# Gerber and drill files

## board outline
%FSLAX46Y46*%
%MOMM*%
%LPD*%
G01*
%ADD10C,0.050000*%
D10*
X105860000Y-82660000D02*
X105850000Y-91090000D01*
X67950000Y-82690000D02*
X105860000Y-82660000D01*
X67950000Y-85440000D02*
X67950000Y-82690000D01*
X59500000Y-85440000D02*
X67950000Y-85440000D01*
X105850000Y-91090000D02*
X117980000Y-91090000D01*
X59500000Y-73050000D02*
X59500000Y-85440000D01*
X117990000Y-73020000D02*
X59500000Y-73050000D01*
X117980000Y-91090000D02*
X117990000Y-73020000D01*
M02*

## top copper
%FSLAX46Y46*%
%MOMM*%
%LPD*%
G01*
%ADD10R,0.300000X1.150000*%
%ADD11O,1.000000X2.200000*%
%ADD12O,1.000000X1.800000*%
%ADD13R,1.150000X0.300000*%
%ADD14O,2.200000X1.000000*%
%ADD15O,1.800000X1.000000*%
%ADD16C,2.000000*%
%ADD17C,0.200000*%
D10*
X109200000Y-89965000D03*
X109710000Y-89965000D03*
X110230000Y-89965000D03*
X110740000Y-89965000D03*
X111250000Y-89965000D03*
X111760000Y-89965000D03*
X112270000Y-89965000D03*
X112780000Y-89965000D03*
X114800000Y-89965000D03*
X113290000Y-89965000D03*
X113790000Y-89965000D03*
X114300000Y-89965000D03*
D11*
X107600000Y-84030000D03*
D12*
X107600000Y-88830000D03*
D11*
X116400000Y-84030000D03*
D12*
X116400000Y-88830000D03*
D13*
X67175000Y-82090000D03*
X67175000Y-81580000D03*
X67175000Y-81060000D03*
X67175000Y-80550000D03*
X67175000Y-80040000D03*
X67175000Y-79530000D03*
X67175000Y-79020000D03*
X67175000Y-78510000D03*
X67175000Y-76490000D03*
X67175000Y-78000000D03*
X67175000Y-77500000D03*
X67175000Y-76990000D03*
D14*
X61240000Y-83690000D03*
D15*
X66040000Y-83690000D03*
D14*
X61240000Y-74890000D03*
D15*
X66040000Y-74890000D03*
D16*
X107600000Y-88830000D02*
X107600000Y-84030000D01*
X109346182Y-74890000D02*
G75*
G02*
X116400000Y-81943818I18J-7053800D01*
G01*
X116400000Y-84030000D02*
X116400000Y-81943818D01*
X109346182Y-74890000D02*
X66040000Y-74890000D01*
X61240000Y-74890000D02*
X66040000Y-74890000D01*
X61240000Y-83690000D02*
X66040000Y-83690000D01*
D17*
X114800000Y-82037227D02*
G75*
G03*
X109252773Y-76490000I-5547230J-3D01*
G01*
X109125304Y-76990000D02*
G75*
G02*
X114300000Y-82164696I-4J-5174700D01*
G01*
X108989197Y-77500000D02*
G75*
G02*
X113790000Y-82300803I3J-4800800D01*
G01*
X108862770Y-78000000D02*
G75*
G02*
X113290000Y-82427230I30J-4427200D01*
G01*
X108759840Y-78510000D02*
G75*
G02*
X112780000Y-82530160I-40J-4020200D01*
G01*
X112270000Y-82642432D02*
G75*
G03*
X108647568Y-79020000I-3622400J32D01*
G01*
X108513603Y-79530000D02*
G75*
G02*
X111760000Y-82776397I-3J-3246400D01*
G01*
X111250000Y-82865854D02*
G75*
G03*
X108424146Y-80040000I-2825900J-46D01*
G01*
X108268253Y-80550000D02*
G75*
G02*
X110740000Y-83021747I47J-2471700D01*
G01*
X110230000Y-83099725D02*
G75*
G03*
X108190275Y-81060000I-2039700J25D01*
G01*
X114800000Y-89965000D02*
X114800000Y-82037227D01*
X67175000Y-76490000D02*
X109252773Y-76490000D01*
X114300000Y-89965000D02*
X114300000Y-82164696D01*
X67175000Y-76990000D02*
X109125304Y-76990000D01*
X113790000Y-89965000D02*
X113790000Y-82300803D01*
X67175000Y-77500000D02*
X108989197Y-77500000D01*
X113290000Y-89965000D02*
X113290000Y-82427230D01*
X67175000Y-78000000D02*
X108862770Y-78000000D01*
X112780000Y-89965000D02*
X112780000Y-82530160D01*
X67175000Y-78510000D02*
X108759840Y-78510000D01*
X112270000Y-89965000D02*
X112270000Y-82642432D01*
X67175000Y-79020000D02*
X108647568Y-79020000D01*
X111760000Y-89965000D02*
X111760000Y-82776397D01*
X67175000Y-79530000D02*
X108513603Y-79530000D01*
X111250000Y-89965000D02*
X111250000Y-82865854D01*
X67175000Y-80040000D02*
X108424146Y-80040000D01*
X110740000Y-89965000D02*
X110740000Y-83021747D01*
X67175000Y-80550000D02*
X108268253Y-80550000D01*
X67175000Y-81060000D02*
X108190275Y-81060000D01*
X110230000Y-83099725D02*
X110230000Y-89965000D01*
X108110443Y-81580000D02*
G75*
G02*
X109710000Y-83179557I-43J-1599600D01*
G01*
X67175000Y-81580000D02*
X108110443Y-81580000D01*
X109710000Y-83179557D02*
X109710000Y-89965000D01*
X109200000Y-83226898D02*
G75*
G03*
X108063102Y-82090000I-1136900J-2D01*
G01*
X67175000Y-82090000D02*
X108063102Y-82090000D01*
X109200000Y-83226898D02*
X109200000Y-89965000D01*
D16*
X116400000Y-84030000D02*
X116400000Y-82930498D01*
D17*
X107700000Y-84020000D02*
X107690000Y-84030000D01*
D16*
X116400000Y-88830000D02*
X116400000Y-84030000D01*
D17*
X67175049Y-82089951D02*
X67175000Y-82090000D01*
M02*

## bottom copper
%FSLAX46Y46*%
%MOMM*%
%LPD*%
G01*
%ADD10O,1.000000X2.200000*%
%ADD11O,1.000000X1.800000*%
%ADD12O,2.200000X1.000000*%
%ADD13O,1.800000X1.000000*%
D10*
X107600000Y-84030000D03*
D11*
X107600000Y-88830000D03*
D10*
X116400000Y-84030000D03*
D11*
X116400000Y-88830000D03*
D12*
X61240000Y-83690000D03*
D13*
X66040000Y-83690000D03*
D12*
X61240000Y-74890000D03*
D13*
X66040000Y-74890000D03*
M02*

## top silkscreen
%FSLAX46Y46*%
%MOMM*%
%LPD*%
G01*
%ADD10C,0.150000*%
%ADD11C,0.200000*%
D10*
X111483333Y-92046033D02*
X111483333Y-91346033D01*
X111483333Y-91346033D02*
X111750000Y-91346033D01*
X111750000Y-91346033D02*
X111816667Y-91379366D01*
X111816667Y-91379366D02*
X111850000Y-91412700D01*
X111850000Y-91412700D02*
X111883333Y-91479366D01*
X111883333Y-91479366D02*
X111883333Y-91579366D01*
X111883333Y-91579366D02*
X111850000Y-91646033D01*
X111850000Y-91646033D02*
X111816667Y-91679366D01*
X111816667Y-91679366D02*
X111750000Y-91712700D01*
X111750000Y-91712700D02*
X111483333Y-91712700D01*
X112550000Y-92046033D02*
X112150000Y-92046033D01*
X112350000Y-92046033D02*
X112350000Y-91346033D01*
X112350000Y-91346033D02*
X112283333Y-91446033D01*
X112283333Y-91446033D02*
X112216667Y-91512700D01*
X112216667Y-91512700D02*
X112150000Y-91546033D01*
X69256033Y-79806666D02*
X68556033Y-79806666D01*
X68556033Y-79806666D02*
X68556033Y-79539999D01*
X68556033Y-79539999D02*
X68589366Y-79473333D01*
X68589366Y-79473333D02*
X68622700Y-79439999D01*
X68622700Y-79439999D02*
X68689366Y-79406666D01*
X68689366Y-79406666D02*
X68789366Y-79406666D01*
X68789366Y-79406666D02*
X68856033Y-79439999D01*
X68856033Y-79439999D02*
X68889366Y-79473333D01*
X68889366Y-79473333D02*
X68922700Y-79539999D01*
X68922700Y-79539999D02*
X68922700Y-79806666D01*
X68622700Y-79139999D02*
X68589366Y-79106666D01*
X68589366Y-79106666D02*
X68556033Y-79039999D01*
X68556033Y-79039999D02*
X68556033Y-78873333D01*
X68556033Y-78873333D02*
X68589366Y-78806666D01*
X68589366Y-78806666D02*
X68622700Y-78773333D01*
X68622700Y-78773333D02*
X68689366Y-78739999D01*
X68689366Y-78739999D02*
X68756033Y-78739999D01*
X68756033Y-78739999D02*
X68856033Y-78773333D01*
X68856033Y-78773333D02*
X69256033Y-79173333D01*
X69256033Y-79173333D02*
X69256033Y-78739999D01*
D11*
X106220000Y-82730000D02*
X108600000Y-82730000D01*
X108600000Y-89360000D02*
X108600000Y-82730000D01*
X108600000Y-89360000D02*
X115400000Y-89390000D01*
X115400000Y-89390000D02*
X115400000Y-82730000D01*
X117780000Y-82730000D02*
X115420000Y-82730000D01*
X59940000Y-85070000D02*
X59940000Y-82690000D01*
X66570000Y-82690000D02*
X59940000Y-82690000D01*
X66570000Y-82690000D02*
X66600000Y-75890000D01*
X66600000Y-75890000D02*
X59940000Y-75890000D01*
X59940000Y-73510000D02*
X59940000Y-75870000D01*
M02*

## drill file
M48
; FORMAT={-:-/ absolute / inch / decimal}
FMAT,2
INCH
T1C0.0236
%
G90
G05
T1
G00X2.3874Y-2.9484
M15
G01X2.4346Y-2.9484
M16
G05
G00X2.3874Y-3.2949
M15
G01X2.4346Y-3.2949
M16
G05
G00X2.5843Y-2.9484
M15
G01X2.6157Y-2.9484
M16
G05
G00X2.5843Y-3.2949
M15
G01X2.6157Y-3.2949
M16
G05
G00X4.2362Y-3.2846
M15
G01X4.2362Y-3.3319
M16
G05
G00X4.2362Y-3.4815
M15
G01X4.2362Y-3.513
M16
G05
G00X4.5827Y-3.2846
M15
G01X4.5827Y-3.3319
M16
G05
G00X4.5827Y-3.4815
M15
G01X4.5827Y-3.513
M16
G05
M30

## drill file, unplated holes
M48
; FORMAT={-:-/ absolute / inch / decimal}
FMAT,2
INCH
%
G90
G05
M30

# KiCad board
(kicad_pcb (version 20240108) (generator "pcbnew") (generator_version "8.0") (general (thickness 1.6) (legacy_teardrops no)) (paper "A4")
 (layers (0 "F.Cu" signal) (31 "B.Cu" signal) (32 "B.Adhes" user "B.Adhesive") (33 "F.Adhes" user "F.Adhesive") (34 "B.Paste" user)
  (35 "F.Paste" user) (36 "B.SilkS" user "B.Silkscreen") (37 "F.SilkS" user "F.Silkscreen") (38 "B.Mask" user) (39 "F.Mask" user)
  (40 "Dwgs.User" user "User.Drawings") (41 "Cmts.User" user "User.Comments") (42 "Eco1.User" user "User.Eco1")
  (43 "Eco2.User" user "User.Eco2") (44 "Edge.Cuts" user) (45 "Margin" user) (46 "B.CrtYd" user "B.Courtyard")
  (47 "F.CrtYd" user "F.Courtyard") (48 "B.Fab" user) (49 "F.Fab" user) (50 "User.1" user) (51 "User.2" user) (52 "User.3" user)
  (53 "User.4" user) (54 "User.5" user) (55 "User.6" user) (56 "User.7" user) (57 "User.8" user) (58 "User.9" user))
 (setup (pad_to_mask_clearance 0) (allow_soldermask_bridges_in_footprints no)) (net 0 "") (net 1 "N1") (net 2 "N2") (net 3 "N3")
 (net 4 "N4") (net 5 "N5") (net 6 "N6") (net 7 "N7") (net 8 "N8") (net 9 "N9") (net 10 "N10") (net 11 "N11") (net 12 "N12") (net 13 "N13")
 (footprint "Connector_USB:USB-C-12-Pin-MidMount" (layer "F.Cu") (at 112 82.73)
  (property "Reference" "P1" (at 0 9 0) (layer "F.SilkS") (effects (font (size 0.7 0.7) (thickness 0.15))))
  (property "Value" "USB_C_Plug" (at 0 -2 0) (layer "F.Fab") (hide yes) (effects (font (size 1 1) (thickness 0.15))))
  (fp_line (start -5.78 0) (end -3.4 0) (stroke (width 0.2) (type solid)) (layer "F.SilkS"))
  (fp_line (start -3.4 6.63) (end -3.4 0) (stroke (width 0.2) (type solid)) (layer "F.SilkS"))
  (fp_line (start -3.4 6.63) (end 3.4 6.66) (stroke (width 0.2) (type solid)) (layer "F.SilkS"))
  (fp_line (start 3.4 6.66) (end 3.4 0) (stroke (width 0.2) (type solid)) (layer "F.SilkS"))
  (fp_line (start 5.78 0) (end 3.42 0) (stroke (width 0.2) (type solid)) (layer "F.SilkS"))
  (pad "A1" smd rect (at -2.8 7.235) (size 0.3 1.15) (layers "F.Cu" "F.Paste" "F.Mask") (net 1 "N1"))
  (pad "A2" smd rect (at -2.29 7.235) (size 0.3 1.15) (layers "F.Cu" "F.Paste" "F.Mask") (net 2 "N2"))
  (pad "A3" smd rect (at -1.77 7.235) (size 0.3 1.15) (layers "F.Cu" "F.Paste" "F.Mask") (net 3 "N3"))
  (pad "A4" smd rect (at -1.26 7.235) (size 0.3 1.15) (layers "F.Cu" "F.Paste" "F.Mask") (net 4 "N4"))
  (pad "A5" smd rect (at -0.75 7.235) (size 0.3 1.15) (layers "F.Cu" "F.Paste" "F.Mask") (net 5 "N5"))
  (pad "A6" smd rect (at -0.24 7.235) (size 0.3 1.15) (layers "F.Cu" "F.Paste" "F.Mask") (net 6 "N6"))
  (pad "A7" smd rect (at 0.27 7.235) (size 0.3 1.15) (layers "F.Cu" "F.Paste" "F.Mask") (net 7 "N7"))
  (pad "A8" smd rect (at 0.78 7.235) (size 0.3 1.15) (layers "F.Cu" "F.Paste" "F.Mask") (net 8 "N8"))
  (pad "B5" smd rect (at 2.8 7.235) (size 0.3 1.15) (layers "F.Cu" "F.Paste" "F.Mask") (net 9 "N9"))
  (pad "B8" smd rect (at 1.29 7.235) (size 0.3 1.15) (layers "F.Cu" "F.Paste" "F.Mask") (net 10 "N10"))
  (pad "B10" smd rect (at 1.79 7.235) (size 0.3 1.15) (layers "F.Cu" "F.Paste" "F.Mask") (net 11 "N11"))
  (pad "B11" smd rect (at 2.3 7.235) (size 0.3 1.15) (layers "F.Cu" "F.Paste" "F.Mask") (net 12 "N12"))
  (pad "S1" thru_hole oval (at -4.4 1.3) (size 1 2.2) (drill oval 0.6 1.8) (layers "*.Cu" "*.Mask") (remove_unused_layers no) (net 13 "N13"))
  (pad "S1" thru_hole oval (at -4.4 6.1) (size 1 1.8) (drill oval 0.6 1.4) (layers "*.Cu" "*.Mask") (remove_unused_layers no) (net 13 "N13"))
  (pad "S1" thru_hole oval (at 4.4 1.3) (size 1 2.2) (drill oval 0.6 1.8) (layers "*.Cu" "*.Mask") (remove_unused_layers no) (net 13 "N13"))
  (pad "S1" thru_hole oval (at 4.4 6.1) (size 1 1.8) (drill oval 0.6 1.4) (layers "*.Cu" "*.Mask") (remove_unused_layers no) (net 13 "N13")))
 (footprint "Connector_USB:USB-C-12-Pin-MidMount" (layer "F.Cu") (at 59.94 79.29 90)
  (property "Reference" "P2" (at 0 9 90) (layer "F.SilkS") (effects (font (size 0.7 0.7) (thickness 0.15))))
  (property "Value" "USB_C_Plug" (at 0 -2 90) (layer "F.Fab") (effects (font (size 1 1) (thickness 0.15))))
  (fp_line (start 5.78 0) (end 3.42 0) (stroke (width 0.2) (type solid)) (layer "F.SilkS"))
  (fp_line (start -5.78 0) (end -3.4 0) (stroke (width 0.2) (type solid)) (layer "F.SilkS"))
  (fp_line (start -3.4 6.63) (end -3.4 0) (stroke (width 0.2) (type solid)) (layer "F.SilkS"))
  (fp_line (start -3.4 6.63) (end 3.4 6.66) (stroke (width 0.2) (type solid)) (layer "F.SilkS"))
  (fp_line (start 3.4 6.66) (end 3.4 0) (stroke (width 0.2) (type solid)) (layer "F.SilkS"))
  (pad "A1" smd rect (at -2.8 7.235 90) (size 0.3 1.15) (layers "F.Cu" "F.Paste" "F.Mask") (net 1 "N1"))
  (pad "A2" smd rect (at -2.29 7.235 90) (size 0.3 1.15) (layers "F.Cu" "F.Paste" "F.Mask") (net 2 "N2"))
  (pad "A3" smd rect (at -1.77 7.235 90) (size 0.3 1.15) (layers "F.Cu" "F.Paste" "F.Mask") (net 3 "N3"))
  (pad "A4" smd rect (at -1.26 7.235 90) (size 0.3 1.15) (layers "F.Cu" "F.Paste" "F.Mask") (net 4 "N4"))
  (pad "A5" smd rect (at -0.75 7.235 90) (size 0.3 1.15) (layers "F.Cu" "F.Paste" "F.Mask") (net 5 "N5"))
  (pad "A6" smd rect (at -0.24 7.235 90) (size 0.3 1.15) (layers "F.Cu" "F.Paste" "F.Mask") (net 6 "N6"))
  (pad "A7" smd rect (at 0.27 7.235 90) (size 0.3 1.15) (layers "F.Cu" "F.Paste" "F.Mask") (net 7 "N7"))
  (pad "A8" smd rect (at 0.78 7.235 90) (size 0.3 1.15) (layers "F.Cu" "F.Paste" "F.Mask") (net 8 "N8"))
  (pad "B5" smd rect (at 2.8 7.235 90) (size 0.3 1.15) (layers "F.Cu" "F.Paste" "F.Mask") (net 9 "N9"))
  (pad "B8" smd rect (at 1.29 7.235 90) (size 0.3 1.15) (layers "F.Cu" "F.Paste" "F.Mask") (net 10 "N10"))
  (pad "B10" smd rect (at 1.79 7.235 90) (size 0.3 1.15) (layers "F.Cu" "F.Paste" "F.Mask") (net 11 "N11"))
  (pad "B11" smd rect (at 2.3 7.235 90) (size 0.3 1.15) (layers "F.Cu" "F.Paste" "F.Mask") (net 12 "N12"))
  (pad "S1" thru_hole oval (at -4.4 1.3 90) (size 1 2.2) (drill oval 0.6 1.8) (layers "*.Cu" "*.Mask") (remove_unused_layers no)
   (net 13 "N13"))
  (pad "S1" thru_hole oval (at -4.4 6.1 90) (size 1 1.8) (drill oval 0.6 1.4) (layers "*.Cu" "*.Mask") (remove_unused_layers no)
   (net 13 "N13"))
  (pad "S1" thru_hole oval (at 4.4 1.3 90) (size 1 2.2) (drill oval 0.6 1.8) (layers "*.Cu" "*.Mask") (remove_unused_layers no)
   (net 13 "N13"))
  (pad "S1" thru_hole oval (at 4.4 6.1 90) (size 1 1.8) (drill oval 0.6 1.4) (layers "*.Cu" "*.Mask") (remove_unused_layers no)
   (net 13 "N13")))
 (gr_line (start 59.5 73.05) (end 59.5 85.44) (stroke (width 0.05) (type default)) (layer "Edge.Cuts"))
 (gr_line (start 105.85 91.09) (end 117.98 91.09) (stroke (width 0.05) (type default)) (layer "Edge.Cuts"))
 (gr_line (start 105.86 82.66) (end 105.85 91.09) (stroke (width 0.05) (type default)) (layer "Edge.Cuts"))
 (gr_line (start 59.5 85.44) (end 67.95 85.44) (stroke (width 0.05) (type default)) (layer "Edge.Cuts"))
 (gr_line (start 117.99 73.02) (end 59.5 73.05) (stroke (width 0.05) (type default)) (layer "Edge.Cuts"))
 (gr_line (start 117.98 91.09) (end 117.99 73.02) (stroke (width 0.05) (type default)) (layer "Edge.Cuts"))
 (gr_line (start 67.95 85.44) (end 67.95 82.69) (stroke (width 0.05) (type default)) (layer "Edge.Cuts"))
 (gr_line (start 67.95 82.69) (end 105.86 82.66) (stroke (width 0.05) (type default)) (layer "Edge.Cuts"))
 (segment (start 67.175049 82.089951) (end 67.175 82.09) (width 0.2) (layer "F.Cu") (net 1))
 (segment (start 67.175 82.09) (end 108.063102 82.09) (width 0.2) (layer "F.Cu") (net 1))
 (segment (start 109.2 83.226898) (end 109.2 89.965) (width 0.2) (layer "F.Cu") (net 1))
 (arc (start 109.2 83.226898) (mid 108.86701 82.42299) (end 108.063102 82.09) (width 0.2) (layer "F.Cu") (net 1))
 (segment (start 67.175 81.58) (end 108.110443 81.58) (width 0.2) (layer "F.Cu") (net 2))
 (segment (start 109.71 83.179557) (end 109.71 89.965) (width 0.2) (layer "F.Cu") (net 2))
 (arc (start 108.110443 81.58) (mid 109.241501 82.048499) (end 109.71 83.179557) (width 0.2) (layer "F.Cu") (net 2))
 (segment (start 67.175 81.06) (end 108.190275 81.06) (width 0.2) (layer "F.Cu") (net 3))
 (segment (start 110.23 83.099725) (end 110.23 89.965) (width 0.2) (layer "F.Cu") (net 3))
 (arc (start 110.23 83.099725) (mid 109.632578 81.657422) (end 108.190275 81.06) (width 0.2) (layer "F.Cu") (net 3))
 (segment (start 110.74 89.965) (end 110.74 83.021747) (width 0.2) (layer "F.Cu") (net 4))
 (segment (start 67.175 80.55) (end 108.268253 80.55) (width 0.2) (layer "F.Cu") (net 4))
 (arc (start 108.268253 80.55) (mid 110.016042 81.273958) (end 110.74 83.021747) (width 0.2) (layer "F.Cu") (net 4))
 (segment (start 111.76 89.965) (end 111.76 82.776397) (width 0.2) (layer "F.Cu") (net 6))
 (segment (start 67.175 79.53) (end 108.513603 79.53) (width 0.2) (layer "F.Cu") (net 6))
 (arc (start 108.513603 79.53) (mid 110.809152 80.480848) (end 111.76 82.776397) (width 0.2) (layer "F.Cu") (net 6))
 (segment (start 111.25 89.965) (end 111.25 82.865854) (width 0.2) (layer "F.Cu") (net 5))
 (segment (start 67.175 80.04) (end 108.424146 80.04) (width 0.2) (layer "F.Cu") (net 5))
 (arc (start 111.25 82.865854) (mid 110.422327 80.867673) (end 108.424146 80.04) (width 0.2) (layer "F.Cu") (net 5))
 (segment (start 67.175 79.02) (end 108.647568 79.02) (width 0.2) (layer "F.Cu") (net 7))
 (segment (start 112.27 89.965) (end 112.27 82.642432) (width 0.2) (layer "F.Cu") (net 7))
 (arc (start 112.27 82.642432) (mid 111.209014 80.080986) (end 108.647568 79.02) (width 0.2) (layer "F.Cu") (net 7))
 (segment (start 114.8 89.965) (end 114.8 82.037227) (width 0.2) (layer "F.Cu") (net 9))
 (segment (start 67.175 76.49) (end 109.252773 76.49) (width 0.2) (layer "F.Cu") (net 9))
 (arc (start 114.8 82.037227) (mid 113.175255 78.114745) (end 109.252773 76.49) (width 0.2) (layer "F.Cu") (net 9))
 (segment (start 107.7 84.02) (end 107.69 84.03) (width 0.2) (layer "F.Cu") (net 13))
 (segment (start 61.24 74.89) (end 66.04 74.89) (width 2) (layer "F.Cu") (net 13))
 (segment (start 116.4 88.83) (end 116.4 84.03) (width 2) (layer "F.Cu") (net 13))
 (segment (start 116.4 84.03) (end 116.4 82.930498) (width 2) (layer "F.Cu") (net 13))
 (segment (start 109.346182 74.89) (end 66.04 74.89) (width 2) (layer "F.Cu") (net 13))
 (segment (start 116.4 84.03) (end 116.4 81.943818) (width 2) (layer "F.Cu") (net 13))
 (segment (start 107.6 88.83) (end 107.6 84.03) (width 2) (layer "F.Cu") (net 13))
 (segment (start 61.24 83.69) (end 66.04 83.69) (width 2) (layer "F.Cu") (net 13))
 (arc (start 109.346182 74.89) (mid 114.333985 76.956015) (end 116.4 81.943818) (width 2) (layer "F.Cu") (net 13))
 (segment (start 67.175 78.51) (end 108.75984 78.51) (width 0.2) (layer "F.Cu") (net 8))
 (segment (start 112.78 89.965) (end 112.78 82.53016) (width 0.2) (layer "F.Cu") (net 8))
 (arc (start 108.75984 78.51) (mid 111.602522 79.687478) (end 112.78 82.53016) (width 0.2) (layer "F.Cu") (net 8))
 (segment (start 114.3 89.965) (end 114.3 82.164696) (width 0.2) (layer "F.Cu") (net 12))
 (segment (start 67.175 76.99) (end 109.125304 76.99) (width 0.2) (layer "F.Cu") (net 12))
 (arc (start 109.125304 76.99) (mid 112.784367 78.505633) (end 114.3 82.164696) (width 0.2) (layer "F.Cu") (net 12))
 (segment (start 113.79 89.965) (end 113.79 82.300803) (width 0.2) (layer "F.Cu") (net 11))
 (segment (start 67.175 77.5) (end 108.989197 77.5) (width 0.2) (layer "F.Cu") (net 11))
 (arc (start 108.989197 77.5) (mid 112.383877 78.906123) (end 113.79 82.300803) (width 0.2) (layer "F.Cu") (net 11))
 (segment (start 113.29 89.965) (end 113.29 82.42723) (width 0.2) (layer "F.Cu") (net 10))
 (segment (start 67.175 78) (end 108.86277 78) (width 0.2) (layer "F.Cu") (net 10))
 (arc (start 108.86277 78) (mid 111.993294 79.296706) (end 113.29 82.42723) (width 0.2) (layer "F.Cu") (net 10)))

